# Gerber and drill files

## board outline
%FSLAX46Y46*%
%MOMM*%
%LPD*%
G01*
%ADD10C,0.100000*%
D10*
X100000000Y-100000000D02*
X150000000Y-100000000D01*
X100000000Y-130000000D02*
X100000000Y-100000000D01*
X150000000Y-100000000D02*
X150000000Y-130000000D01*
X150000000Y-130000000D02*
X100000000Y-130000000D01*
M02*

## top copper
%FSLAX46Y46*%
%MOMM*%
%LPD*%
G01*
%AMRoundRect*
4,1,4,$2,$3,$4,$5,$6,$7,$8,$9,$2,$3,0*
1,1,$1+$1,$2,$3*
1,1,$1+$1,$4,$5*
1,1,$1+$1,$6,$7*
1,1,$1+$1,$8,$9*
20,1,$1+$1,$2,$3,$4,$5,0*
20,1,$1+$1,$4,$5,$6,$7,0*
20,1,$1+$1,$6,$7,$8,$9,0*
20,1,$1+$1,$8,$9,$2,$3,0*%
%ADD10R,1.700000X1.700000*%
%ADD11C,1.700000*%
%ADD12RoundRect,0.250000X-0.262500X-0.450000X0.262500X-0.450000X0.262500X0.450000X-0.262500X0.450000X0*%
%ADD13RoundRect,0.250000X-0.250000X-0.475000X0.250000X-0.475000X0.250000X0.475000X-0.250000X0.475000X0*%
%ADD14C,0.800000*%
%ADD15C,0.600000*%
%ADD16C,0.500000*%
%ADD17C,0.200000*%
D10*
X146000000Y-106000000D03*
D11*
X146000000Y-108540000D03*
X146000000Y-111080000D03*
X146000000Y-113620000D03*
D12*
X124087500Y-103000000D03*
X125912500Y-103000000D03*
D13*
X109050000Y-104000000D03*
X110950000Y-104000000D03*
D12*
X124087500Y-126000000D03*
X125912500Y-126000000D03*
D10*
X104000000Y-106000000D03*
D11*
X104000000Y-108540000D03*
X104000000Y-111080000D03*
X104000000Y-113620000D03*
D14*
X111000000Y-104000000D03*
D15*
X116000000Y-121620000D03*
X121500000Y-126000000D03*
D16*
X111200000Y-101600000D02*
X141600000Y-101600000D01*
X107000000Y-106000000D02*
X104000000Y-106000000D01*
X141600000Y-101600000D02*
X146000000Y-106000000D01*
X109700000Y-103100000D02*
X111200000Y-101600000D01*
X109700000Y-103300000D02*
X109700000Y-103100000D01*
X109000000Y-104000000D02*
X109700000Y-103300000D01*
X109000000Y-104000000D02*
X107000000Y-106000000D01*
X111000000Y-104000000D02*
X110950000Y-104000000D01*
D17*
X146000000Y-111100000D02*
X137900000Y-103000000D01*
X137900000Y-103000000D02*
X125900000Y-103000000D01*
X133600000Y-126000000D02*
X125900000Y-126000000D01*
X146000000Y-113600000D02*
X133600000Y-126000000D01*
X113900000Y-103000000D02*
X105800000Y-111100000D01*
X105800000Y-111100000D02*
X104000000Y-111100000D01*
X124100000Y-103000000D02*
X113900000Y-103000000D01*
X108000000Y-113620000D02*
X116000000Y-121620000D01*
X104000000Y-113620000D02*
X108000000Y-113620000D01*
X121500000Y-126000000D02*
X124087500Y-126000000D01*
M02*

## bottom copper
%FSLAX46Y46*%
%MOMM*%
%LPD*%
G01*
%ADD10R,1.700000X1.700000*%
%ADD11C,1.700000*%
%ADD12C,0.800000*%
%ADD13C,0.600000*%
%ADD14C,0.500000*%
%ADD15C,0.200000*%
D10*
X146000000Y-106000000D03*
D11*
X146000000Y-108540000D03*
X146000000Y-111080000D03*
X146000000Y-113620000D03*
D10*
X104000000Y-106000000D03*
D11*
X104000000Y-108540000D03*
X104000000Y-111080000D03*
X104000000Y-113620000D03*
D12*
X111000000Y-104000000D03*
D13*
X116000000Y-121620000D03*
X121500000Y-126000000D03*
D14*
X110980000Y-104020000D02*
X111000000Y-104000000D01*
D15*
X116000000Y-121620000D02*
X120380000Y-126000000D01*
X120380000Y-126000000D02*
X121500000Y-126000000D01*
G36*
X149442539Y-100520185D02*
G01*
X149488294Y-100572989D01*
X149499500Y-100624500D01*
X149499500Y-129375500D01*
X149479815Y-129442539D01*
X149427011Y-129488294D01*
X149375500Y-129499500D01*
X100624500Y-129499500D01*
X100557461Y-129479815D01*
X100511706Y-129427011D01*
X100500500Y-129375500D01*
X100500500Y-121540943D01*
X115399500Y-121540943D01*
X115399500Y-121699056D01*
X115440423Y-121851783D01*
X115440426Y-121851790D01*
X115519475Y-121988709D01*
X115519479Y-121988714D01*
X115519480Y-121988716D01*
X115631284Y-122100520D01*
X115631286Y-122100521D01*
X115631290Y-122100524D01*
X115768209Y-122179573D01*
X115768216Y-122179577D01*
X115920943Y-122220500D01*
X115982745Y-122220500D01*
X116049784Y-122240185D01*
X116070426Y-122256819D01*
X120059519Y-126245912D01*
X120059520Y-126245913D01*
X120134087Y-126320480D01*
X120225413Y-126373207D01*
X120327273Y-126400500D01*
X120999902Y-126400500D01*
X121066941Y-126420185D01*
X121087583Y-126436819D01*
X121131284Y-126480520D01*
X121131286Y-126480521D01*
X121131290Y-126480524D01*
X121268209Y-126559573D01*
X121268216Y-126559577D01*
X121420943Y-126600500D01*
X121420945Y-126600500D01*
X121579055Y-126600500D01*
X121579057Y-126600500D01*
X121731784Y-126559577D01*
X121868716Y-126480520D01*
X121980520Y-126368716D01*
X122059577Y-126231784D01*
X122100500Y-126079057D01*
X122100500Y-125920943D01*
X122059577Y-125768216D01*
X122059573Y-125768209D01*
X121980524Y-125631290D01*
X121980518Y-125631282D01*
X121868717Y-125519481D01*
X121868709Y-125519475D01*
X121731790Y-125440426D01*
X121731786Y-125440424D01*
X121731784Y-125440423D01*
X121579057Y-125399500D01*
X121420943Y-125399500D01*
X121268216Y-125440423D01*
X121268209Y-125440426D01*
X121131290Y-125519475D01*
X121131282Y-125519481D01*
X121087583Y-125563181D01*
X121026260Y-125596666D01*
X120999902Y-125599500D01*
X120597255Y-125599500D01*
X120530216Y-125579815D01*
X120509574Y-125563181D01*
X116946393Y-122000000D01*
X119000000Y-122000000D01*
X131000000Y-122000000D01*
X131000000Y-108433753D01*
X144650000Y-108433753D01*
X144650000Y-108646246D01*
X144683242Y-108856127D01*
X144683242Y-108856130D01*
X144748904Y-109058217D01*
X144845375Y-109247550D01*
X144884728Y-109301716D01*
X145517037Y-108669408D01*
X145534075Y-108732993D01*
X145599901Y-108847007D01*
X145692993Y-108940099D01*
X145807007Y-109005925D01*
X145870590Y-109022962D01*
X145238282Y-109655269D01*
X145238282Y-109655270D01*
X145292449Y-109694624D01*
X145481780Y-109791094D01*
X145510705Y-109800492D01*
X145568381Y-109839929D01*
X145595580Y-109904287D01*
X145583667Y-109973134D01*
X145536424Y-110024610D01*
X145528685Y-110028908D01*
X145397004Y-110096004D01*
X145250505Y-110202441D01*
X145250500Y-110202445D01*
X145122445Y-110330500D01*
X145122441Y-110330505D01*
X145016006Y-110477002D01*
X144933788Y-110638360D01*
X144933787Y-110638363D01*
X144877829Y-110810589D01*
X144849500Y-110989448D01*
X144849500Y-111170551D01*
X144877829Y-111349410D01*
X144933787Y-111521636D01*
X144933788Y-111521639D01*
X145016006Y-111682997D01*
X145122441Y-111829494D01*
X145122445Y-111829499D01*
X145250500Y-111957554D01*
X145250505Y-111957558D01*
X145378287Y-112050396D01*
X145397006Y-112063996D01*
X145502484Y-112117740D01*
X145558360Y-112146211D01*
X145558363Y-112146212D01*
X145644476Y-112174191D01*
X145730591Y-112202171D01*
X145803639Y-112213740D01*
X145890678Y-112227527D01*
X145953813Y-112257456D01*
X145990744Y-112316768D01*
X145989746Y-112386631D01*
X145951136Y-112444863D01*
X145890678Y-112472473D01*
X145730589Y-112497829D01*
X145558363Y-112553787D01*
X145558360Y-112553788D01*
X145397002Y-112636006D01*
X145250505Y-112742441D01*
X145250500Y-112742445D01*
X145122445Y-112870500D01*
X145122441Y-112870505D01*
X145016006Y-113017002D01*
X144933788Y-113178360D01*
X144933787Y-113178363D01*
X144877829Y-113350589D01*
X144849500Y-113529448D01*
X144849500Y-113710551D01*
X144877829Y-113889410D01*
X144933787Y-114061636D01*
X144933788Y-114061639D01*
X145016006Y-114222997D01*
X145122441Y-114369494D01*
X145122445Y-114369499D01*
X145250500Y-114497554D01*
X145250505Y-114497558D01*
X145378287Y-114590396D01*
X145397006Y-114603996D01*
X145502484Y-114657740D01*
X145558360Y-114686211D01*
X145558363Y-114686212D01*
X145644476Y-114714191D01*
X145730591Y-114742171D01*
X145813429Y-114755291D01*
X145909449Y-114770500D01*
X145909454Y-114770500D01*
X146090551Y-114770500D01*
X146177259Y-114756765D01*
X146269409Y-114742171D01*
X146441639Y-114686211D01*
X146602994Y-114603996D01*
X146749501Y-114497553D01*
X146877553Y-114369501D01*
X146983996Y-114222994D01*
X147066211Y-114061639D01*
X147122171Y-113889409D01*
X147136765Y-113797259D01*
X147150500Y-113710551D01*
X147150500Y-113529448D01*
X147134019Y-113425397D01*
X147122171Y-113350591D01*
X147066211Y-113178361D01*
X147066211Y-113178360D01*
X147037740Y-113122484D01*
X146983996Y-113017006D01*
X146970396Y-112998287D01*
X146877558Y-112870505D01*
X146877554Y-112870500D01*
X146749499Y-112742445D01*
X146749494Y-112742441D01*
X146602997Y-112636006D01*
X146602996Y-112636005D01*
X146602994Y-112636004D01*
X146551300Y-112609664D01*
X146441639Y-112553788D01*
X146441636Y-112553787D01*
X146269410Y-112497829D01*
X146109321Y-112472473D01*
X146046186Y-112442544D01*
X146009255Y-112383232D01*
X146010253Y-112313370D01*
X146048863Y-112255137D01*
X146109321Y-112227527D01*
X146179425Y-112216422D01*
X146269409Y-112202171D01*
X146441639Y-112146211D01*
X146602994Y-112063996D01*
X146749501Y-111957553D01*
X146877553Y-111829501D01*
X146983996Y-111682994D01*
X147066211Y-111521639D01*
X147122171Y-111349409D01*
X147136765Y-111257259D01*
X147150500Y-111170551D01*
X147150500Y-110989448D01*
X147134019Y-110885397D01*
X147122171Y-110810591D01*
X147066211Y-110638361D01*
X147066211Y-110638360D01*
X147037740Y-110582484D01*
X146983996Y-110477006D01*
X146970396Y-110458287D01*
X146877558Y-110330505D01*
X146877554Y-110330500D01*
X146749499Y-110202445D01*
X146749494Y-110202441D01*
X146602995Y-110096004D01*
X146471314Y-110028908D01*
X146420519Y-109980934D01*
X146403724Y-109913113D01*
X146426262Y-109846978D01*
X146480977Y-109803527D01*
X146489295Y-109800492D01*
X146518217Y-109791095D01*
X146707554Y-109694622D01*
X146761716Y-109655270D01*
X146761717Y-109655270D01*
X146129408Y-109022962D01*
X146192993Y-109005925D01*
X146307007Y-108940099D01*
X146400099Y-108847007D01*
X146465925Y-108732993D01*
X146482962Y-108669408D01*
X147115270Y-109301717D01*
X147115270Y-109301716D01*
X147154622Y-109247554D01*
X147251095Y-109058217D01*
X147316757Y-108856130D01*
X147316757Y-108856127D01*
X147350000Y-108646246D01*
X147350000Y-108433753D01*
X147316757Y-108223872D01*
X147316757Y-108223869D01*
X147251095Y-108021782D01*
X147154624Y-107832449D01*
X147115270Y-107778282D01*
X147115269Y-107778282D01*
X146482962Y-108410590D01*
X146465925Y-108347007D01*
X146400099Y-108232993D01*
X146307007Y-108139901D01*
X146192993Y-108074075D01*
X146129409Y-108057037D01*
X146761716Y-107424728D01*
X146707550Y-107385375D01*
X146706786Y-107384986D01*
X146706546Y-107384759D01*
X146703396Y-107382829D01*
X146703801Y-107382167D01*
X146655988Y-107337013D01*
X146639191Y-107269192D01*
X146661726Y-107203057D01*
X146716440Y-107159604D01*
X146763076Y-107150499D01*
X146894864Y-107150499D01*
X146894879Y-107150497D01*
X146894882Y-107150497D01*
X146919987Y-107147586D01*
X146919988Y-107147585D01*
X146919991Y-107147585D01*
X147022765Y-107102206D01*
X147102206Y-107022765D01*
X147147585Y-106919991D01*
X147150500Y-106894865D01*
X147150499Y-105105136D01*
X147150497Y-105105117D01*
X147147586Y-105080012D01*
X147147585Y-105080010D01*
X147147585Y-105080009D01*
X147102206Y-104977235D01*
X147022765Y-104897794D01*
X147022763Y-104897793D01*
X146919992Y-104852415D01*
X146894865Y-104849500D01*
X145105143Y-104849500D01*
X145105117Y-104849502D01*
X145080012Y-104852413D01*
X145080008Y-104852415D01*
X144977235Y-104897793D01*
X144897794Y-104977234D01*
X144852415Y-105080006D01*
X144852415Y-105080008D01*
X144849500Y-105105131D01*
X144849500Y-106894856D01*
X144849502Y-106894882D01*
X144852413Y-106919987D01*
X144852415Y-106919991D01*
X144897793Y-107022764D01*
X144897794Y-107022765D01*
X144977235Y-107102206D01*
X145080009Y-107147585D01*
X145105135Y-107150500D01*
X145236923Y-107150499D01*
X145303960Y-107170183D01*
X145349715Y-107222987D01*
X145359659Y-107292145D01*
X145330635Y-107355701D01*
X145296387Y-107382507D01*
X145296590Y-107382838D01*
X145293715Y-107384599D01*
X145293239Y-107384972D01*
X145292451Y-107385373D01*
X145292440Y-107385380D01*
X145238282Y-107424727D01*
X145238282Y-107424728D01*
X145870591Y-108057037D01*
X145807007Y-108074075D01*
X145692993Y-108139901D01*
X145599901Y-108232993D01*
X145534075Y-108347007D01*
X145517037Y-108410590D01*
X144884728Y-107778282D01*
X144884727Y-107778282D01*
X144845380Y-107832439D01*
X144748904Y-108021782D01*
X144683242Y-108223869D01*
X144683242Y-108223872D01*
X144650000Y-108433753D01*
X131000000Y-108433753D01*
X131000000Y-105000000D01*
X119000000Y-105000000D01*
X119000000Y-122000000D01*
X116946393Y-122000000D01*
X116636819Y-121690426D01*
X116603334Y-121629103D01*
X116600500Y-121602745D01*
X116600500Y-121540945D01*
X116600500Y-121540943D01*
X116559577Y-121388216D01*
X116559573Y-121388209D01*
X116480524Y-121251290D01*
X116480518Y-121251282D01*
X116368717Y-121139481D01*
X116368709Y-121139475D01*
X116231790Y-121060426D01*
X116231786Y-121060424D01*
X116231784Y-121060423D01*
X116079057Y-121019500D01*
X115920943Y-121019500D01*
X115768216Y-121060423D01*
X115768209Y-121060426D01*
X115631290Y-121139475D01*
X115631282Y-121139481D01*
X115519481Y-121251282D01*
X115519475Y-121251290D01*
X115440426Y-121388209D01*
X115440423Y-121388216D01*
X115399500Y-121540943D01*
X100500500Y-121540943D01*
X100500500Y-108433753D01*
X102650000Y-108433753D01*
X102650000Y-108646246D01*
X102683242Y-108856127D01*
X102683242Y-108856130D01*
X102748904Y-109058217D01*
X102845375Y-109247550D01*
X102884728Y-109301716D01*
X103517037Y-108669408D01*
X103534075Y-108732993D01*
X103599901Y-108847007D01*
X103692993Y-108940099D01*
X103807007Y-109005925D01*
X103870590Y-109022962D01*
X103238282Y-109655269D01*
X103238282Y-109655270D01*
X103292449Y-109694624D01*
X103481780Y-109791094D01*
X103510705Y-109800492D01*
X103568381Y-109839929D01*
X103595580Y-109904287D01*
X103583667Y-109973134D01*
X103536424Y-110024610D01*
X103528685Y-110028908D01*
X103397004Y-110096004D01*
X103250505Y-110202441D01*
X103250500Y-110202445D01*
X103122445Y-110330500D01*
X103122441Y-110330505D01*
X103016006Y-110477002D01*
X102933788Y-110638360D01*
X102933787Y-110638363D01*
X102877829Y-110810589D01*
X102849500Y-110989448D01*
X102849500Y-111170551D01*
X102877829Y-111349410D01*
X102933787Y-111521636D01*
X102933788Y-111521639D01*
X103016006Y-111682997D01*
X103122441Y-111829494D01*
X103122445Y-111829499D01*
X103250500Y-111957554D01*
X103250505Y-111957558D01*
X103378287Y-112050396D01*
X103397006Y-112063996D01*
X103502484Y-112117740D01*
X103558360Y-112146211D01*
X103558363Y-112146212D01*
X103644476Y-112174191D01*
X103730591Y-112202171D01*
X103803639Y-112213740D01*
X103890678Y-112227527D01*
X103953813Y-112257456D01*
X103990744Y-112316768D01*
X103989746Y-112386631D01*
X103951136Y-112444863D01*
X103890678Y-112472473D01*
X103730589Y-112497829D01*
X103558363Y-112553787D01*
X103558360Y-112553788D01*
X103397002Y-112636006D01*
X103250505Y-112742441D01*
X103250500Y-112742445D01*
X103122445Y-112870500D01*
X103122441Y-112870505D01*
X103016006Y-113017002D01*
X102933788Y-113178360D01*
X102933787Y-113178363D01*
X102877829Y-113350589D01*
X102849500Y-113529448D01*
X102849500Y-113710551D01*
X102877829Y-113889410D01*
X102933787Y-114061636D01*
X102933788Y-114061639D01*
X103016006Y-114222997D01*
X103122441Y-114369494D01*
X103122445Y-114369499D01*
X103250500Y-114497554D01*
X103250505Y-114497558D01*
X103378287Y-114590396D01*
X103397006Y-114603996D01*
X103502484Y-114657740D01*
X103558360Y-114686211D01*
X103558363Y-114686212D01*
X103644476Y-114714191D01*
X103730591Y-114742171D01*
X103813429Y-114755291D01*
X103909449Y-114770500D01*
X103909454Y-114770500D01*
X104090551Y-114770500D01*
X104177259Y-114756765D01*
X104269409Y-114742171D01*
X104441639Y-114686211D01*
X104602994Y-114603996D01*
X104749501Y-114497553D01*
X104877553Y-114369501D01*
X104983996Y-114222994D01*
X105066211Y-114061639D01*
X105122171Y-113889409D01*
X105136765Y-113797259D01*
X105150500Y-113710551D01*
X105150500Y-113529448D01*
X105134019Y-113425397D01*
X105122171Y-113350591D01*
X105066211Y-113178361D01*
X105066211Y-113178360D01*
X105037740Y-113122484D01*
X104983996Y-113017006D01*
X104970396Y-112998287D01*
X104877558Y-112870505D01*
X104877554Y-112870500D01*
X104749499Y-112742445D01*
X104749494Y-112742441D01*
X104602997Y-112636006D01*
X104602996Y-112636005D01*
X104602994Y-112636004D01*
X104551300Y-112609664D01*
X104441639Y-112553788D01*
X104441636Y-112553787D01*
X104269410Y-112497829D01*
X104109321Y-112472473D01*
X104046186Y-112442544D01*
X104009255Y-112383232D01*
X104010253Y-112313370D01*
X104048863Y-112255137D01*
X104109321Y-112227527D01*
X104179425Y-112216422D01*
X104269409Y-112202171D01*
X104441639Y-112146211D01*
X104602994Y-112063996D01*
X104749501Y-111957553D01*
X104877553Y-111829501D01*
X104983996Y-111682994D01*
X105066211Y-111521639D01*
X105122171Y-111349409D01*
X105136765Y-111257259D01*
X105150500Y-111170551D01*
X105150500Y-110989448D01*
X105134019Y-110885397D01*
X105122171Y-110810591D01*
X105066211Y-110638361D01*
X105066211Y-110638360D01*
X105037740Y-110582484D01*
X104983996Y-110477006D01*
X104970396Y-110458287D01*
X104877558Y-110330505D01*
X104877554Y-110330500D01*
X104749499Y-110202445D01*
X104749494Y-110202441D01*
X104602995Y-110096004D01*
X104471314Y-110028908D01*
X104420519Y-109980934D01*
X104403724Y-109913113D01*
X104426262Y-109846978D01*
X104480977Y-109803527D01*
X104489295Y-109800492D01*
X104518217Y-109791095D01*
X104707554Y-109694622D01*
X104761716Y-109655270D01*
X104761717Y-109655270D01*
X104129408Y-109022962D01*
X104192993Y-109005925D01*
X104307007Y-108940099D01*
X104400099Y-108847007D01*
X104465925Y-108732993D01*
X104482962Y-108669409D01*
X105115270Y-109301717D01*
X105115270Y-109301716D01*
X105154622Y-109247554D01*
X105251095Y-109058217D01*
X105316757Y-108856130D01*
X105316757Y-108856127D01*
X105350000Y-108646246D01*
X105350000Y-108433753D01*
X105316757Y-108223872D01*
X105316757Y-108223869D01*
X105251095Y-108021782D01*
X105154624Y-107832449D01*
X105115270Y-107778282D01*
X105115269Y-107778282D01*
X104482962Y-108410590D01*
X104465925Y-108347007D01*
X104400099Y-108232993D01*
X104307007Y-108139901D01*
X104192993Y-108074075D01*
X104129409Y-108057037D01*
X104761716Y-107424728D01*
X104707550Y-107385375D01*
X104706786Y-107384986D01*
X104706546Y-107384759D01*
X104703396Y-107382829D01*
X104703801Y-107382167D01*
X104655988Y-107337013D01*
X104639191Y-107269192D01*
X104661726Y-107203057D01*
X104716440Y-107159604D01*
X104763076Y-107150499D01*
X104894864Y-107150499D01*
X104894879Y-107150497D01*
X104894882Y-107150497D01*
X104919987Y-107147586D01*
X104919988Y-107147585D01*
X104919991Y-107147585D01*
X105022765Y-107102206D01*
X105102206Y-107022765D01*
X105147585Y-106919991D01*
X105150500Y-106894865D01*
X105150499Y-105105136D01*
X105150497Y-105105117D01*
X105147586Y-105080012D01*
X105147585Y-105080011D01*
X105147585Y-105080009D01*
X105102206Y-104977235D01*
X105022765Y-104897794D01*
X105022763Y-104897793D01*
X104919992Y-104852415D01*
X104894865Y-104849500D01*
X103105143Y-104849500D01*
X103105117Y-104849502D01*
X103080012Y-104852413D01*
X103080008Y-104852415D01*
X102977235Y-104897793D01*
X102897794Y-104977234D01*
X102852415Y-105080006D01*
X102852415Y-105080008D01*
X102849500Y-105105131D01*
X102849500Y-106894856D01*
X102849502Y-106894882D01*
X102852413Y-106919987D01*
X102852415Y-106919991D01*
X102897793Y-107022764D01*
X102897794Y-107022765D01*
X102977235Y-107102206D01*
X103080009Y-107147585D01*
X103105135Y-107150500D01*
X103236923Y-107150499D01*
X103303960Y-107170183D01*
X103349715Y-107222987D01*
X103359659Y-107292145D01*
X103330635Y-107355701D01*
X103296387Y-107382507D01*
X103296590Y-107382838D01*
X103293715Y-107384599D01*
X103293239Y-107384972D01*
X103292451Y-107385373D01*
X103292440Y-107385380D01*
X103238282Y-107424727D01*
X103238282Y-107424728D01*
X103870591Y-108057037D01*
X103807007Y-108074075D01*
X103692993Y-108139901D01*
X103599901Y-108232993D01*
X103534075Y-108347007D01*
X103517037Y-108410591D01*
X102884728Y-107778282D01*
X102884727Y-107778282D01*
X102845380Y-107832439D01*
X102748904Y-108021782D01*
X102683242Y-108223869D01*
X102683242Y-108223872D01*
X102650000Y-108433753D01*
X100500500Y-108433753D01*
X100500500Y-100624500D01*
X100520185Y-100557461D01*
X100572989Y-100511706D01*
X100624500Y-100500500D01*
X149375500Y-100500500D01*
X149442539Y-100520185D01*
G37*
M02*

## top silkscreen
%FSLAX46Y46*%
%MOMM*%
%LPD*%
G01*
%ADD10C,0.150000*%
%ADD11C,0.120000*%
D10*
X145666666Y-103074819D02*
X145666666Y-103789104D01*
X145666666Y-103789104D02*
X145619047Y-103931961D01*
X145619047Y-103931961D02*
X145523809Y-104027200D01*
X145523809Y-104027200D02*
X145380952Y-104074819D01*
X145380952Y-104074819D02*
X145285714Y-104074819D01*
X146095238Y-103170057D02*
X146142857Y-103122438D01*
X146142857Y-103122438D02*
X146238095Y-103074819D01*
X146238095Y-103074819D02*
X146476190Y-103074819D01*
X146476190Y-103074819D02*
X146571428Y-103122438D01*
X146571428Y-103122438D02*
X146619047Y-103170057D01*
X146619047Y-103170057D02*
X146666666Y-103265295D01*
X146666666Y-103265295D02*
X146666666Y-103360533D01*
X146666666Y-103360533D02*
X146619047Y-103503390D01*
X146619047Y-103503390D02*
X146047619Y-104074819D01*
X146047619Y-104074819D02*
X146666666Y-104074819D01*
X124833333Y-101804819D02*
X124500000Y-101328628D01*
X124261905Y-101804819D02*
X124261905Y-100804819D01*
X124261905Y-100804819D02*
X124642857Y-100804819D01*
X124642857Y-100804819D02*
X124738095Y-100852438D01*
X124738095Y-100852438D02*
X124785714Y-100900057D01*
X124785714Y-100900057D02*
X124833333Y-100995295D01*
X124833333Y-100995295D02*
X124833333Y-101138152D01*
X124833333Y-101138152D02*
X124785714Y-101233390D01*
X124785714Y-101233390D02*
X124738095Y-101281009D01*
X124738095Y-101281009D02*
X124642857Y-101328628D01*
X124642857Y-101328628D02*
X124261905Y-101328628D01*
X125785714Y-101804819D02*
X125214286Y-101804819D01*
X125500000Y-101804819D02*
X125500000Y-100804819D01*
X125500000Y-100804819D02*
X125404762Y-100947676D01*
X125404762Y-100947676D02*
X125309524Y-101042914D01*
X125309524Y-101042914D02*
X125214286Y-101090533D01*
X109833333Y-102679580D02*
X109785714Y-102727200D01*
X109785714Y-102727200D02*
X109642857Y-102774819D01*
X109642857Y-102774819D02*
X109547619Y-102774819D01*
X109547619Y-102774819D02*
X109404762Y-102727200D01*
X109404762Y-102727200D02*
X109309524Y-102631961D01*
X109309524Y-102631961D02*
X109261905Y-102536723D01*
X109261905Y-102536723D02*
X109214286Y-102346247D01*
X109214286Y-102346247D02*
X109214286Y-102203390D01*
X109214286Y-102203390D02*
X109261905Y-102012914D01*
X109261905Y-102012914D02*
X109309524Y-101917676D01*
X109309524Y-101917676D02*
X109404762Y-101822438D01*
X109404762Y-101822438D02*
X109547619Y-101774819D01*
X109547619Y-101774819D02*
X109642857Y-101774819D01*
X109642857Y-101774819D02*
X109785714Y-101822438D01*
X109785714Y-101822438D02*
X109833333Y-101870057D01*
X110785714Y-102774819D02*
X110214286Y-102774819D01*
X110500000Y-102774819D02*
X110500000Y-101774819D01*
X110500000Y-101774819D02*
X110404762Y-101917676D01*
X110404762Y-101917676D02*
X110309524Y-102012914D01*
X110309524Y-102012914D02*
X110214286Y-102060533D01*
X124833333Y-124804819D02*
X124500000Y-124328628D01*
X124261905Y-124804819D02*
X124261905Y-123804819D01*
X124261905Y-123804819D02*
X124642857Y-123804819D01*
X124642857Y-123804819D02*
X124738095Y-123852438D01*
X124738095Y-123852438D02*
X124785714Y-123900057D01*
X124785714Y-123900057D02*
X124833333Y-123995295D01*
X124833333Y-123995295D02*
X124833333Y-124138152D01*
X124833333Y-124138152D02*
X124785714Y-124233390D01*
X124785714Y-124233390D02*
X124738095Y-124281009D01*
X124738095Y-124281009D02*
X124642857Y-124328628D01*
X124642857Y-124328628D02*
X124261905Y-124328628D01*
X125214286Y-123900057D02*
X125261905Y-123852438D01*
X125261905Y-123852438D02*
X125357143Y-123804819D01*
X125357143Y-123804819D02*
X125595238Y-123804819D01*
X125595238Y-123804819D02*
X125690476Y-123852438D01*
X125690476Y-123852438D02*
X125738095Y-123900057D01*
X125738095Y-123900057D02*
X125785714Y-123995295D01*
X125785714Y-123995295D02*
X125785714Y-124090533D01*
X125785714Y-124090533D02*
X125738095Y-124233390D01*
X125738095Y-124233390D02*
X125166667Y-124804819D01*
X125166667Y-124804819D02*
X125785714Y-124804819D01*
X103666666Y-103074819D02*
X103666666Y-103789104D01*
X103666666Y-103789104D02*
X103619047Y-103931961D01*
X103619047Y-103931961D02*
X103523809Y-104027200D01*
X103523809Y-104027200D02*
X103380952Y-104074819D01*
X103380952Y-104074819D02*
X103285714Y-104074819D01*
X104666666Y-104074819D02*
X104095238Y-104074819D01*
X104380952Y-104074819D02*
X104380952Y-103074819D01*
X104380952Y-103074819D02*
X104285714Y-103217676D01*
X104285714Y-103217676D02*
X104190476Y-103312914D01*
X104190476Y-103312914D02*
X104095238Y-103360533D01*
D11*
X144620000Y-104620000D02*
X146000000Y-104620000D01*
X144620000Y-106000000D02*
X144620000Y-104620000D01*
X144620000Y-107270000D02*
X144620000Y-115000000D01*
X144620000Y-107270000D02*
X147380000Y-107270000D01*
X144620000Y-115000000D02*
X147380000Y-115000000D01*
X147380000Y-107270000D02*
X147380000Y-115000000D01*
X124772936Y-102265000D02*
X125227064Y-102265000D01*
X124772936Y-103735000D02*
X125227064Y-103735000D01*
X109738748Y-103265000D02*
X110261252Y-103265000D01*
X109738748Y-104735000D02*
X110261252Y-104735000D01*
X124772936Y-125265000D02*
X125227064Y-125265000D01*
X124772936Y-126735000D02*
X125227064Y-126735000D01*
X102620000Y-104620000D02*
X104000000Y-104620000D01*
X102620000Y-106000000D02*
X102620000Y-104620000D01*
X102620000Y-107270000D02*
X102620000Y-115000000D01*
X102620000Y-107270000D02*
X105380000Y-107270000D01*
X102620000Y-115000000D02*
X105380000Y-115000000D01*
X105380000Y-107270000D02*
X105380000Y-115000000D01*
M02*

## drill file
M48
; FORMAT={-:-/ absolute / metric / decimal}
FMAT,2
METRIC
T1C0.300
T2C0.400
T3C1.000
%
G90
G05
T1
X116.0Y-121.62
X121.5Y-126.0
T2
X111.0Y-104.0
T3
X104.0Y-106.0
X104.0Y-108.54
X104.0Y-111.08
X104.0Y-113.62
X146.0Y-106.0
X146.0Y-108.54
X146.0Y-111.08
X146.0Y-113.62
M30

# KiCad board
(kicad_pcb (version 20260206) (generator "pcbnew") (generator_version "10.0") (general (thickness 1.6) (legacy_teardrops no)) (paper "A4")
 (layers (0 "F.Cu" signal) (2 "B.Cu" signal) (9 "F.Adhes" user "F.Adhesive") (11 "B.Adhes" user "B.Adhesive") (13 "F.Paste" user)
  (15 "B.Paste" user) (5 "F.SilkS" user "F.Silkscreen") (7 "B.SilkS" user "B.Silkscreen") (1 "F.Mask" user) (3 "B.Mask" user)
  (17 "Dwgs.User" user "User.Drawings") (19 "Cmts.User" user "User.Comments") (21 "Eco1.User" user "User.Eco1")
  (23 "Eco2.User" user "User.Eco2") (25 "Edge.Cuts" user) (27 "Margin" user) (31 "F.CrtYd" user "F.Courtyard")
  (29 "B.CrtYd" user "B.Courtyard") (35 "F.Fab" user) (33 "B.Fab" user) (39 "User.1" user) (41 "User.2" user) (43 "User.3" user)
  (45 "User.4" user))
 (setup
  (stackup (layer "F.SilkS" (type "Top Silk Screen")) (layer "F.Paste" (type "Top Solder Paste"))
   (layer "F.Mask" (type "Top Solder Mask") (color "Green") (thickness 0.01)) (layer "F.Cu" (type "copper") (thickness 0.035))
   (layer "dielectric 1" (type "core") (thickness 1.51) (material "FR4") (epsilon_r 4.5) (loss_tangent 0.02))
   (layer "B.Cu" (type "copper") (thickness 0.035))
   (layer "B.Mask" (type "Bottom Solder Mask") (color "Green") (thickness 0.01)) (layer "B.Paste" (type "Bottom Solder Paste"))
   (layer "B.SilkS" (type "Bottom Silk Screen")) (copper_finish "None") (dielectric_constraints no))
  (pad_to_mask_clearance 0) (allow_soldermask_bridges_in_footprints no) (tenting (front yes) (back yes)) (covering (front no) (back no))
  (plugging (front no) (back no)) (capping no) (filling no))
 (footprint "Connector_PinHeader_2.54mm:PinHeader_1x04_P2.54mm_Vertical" (layer "F.Cu") (at 146 106)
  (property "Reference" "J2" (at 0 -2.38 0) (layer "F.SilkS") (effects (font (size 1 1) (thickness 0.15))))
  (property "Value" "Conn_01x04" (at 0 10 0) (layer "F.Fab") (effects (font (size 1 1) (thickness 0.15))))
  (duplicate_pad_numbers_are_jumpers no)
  (fp_line (start -1.38 -1.38) (end 0 -1.38) (stroke (width 0.12) (type solid)) (layer "F.SilkS"))
  (fp_line (start -1.38 0) (end -1.38 -1.38) (stroke (width 0.12) (type solid)) (layer "F.SilkS"))
  (fp_line (start -1.38 1.27) (end -1.38 9) (stroke (width 0.12) (type solid)) (layer "F.SilkS"))
  (fp_line (start -1.38 1.27) (end 1.38 1.27) (stroke (width 0.12) (type solid)) (layer "F.SilkS"))
  (fp_line (start -1.38 9) (end 1.38 9) (stroke (width 0.12) (type solid)) (layer "F.SilkS"))
  (fp_line (start 1.38 1.27) (end 1.38 9) (stroke (width 0.12) (type solid)) (layer "F.SilkS"))
  (pad "1" thru_hole rect (at 0 0) (size 1.7 1.7) (drill 1) (layers "*.Cu" "*.Mask") (remove_unused_layers no) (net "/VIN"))
  (pad "2" thru_hole circle (at 0 2.54) (size 1.7 1.7) (drill 1) (layers "*.Cu" "*.Mask") (remove_unused_layers no) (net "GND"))
  (pad "3" thru_hole circle (at 0 5.08) (size 1.7 1.7) (drill 1) (layers "*.Cu" "*.Mask") (remove_unused_layers no) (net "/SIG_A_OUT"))
  (pad "4" thru_hole circle (at 0 7.62) (size 1.7 1.7) (drill 1) (layers "*.Cu" "*.Mask") (remove_unused_layers no) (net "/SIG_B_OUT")))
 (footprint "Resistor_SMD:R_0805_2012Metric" (layer "F.Cu") (at 125 103)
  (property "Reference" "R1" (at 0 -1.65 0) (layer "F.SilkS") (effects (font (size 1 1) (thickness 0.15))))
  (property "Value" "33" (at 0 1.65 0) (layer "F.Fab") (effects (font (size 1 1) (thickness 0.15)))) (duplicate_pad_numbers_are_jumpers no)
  (fp_line (start -0.227064 -0.735) (end 0.227064 -0.735) (stroke (width 0.12) (type solid)) (layer "F.SilkS"))
  (fp_line (start -0.227064 0.735) (end 0.227064 0.735) (stroke (width 0.12) (type solid)) (layer "F.SilkS"))
  (pad "1" smd roundrect (at -0.9125 0) (size 1.025 1.4) (layers "F.Cu" "F.Mask" "F.Paste") (roundrect_rratio 0.243902) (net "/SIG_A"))
  (pad "2" smd roundrect (at 0.9125 0) (size 1.025 1.4) (layers "F.Cu" "F.Mask" "F.Paste") (roundrect_rratio 0.243902) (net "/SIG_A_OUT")))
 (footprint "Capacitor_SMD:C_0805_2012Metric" (layer "F.Cu") (at 110 104)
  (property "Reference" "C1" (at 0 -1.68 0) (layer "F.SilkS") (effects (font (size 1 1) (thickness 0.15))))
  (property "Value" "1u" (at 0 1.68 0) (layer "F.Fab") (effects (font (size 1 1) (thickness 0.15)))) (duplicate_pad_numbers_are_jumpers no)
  (fp_line (start -0.261252 -0.735) (end 0.261252 -0.735) (stroke (width 0.12) (type solid)) (layer "F.SilkS"))
  (fp_line (start -0.261252 0.735) (end 0.261252 0.735) (stroke (width 0.12) (type solid)) (layer "F.SilkS"))
  (pad "1" smd roundrect (at -0.95 0) (size 1 1.45) (layers "F.Cu" "F.Mask" "F.Paste") (roundrect_rratio 0.25) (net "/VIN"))
  (pad "2" smd roundrect (at 0.95 0) (size 1 1.45) (layers "F.Cu" "F.Mask" "F.Paste") (roundrect_rratio 0.25) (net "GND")))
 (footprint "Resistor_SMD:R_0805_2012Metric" (layer "F.Cu") (at 125 126)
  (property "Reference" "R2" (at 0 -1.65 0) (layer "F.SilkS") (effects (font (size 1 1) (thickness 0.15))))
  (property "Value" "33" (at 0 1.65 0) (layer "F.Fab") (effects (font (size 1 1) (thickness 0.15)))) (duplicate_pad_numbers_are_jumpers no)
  (fp_line (start -0.227064 -0.735) (end 0.227064 -0.735) (stroke (width 0.12) (type solid)) (layer "F.SilkS"))
  (fp_line (start -0.227064 0.735) (end 0.227064 0.735) (stroke (width 0.12) (type solid)) (layer "F.SilkS"))
  (pad "1" smd roundrect (at -0.9125 0) (size 1.025 1.4) (layers "F.Cu" "F.Mask" "F.Paste") (roundrect_rratio 0.243902) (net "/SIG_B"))
  (pad "2" smd roundrect (at 0.9125 0) (size 1.025 1.4) (layers "F.Cu" "F.Mask" "F.Paste") (roundrect_rratio 0.243902) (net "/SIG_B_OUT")))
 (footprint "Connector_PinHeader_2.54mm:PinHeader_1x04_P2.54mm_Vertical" (layer "F.Cu") (at 104 106)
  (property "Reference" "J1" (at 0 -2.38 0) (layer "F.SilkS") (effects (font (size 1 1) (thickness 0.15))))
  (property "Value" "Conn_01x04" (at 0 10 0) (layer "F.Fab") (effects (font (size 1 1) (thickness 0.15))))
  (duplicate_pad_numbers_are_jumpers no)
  (fp_line (start -1.38 -1.38) (end 0 -1.38) (stroke (width 0.12) (type solid)) (layer "F.SilkS"))
  (fp_line (start -1.38 0) (end -1.38 -1.38) (stroke (width 0.12) (type solid)) (layer "F.SilkS"))
  (fp_line (start -1.38 1.27) (end -1.38 9) (stroke (width 0.12) (type solid)) (layer "F.SilkS"))
  (fp_line (start -1.38 1.27) (end 1.38 1.27) (stroke (width 0.12) (type solid)) (layer "F.SilkS"))
  (fp_line (start -1.38 9) (end 1.38 9) (stroke (width 0.12) (type solid)) (layer "F.SilkS"))
  (fp_line (start 1.38 1.27) (end 1.38 9) (stroke (width 0.12) (type solid)) (layer "F.SilkS"))
  (pad "1" thru_hole rect (at 0 0) (size 1.7 1.7) (drill 1) (layers "*.Cu" "*.Mask") (remove_unused_layers no) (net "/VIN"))
  (pad "2" thru_hole circle (at 0 2.54) (size 1.7 1.7) (drill 1) (layers "*.Cu" "*.Mask") (remove_unused_layers no) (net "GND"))
  (pad "3" thru_hole circle (at 0 5.08) (size 1.7 1.7) (drill 1) (layers "*.Cu" "*.Mask") (remove_unused_layers no) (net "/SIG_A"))
  (pad "4" thru_hole circle (at 0 7.62) (size 1.7 1.7) (drill 1) (layers "*.Cu" "*.Mask") (remove_unused_layers no) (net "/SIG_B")))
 (gr_line (start 100 100) (end 150 100) (stroke (width 0.1) (type default)) (layer "Edge.Cuts"))
 (gr_line (start 100 130) (end 100 100) (stroke (width 0.1) (type default)) (layer "Edge.Cuts"))
 (gr_line (start 150 100) (end 150 130) (stroke (width 0.1) (type default)) (layer "Edge.Cuts"))
 (gr_line (start 150 130) (end 100 130) (stroke (width 0.1) (type default)) (layer "Edge.Cuts"))
 (segment (start 111.2 101.6) (end 141.6 101.6) (width 0.5) (layer "F.Cu") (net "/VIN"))
 (segment (start 107 106) (end 104 106) (width 0.5) (layer "F.Cu") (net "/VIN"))
 (segment (start 141.6 101.6) (end 146 106) (width 0.5) (layer "F.Cu") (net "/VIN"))
 (segment (start 109.7 103.1) (end 111.2 101.6) (width 0.5) (layer "F.Cu") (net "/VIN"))
 (segment (start 109.7 103.3) (end 109.7 103.1) (width 0.5) (layer "F.Cu") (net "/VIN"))
 (segment (start 109 104) (end 109.7 103.3) (width 0.5) (layer "F.Cu") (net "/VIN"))
 (segment (start 109 104) (end 107 106) (width 0.5) (layer "F.Cu") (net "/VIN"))
 (segment (start 111 104) (end 110.95 104) (width 0.5) (layer "F.Cu") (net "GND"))
 (via (at 111 104) (size 0.8) (drill 0.4) (layers "F.Cu" "B.Cu") (capping yes) (filling yes) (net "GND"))
 (segment (start 110.98 104.02) (end 111 104) (width 0.5) (layer "B.Cu") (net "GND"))
 (segment (start 146 111.1) (end 137.9 103) (width 0.2) (layer "F.Cu") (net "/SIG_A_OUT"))
 (segment (start 137.9 103) (end 125.9 103) (width 0.2) (layer "F.Cu") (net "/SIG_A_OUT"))
 (segment (start 133.6 126) (end 125.9 126) (width 0.2) (layer "F.Cu") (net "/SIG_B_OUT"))
 (segment (start 146 113.6) (end 133.6 126) (width 0.2) (layer "F.Cu") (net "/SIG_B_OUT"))
 (segment (start 113.9 103) (end 105.8 111.1) (width 0.2) (layer "F.Cu") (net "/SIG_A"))
 (segment (start 105.8 111.1) (end 104 111.1) (width 0.2) (layer "F.Cu") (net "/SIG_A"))
 (segment (start 124.1 103) (end 113.9 103) (width 0.2) (layer "F.Cu") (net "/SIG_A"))
 (segment (start 108 113.62) (end 116 121.62) (width 0.2) (locked yes) (layer "F.Cu") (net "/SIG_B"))
 (segment (start 104 113.62) (end 108 113.62) (width 0.2) (locked yes) (layer "F.Cu") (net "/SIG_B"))
 (segment (start 121.5 126) (end 124.0875 126) (width 0.2) (locked yes) (layer "F.Cu") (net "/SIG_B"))
 (via (at 116 121.62) (size 0.6) (drill 0.3) (layers "F.Cu" "B.Cu") (locked yes) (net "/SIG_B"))
 (via (at 121.5 126) (size 0.6) (drill 0.3) (layers "F.Cu" "B.Cu") (locked yes) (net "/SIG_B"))
 (segment (start 116 121.62) (end 120.38 126) (width 0.2) (locked yes) (layer "B.Cu") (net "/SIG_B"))
 (segment (start 120.38 126) (end 121.5 126) (width 0.2) (locked yes) (layer "B.Cu") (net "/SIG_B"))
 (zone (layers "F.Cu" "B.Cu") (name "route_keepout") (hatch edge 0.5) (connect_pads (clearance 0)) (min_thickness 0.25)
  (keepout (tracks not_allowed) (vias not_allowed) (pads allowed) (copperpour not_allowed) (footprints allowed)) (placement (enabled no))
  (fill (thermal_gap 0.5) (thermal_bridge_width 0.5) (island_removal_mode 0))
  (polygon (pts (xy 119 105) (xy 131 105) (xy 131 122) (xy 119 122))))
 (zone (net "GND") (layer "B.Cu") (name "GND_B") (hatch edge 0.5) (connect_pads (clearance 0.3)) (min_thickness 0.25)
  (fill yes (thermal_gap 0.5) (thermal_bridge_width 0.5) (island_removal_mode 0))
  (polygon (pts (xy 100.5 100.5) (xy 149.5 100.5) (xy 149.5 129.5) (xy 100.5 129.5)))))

